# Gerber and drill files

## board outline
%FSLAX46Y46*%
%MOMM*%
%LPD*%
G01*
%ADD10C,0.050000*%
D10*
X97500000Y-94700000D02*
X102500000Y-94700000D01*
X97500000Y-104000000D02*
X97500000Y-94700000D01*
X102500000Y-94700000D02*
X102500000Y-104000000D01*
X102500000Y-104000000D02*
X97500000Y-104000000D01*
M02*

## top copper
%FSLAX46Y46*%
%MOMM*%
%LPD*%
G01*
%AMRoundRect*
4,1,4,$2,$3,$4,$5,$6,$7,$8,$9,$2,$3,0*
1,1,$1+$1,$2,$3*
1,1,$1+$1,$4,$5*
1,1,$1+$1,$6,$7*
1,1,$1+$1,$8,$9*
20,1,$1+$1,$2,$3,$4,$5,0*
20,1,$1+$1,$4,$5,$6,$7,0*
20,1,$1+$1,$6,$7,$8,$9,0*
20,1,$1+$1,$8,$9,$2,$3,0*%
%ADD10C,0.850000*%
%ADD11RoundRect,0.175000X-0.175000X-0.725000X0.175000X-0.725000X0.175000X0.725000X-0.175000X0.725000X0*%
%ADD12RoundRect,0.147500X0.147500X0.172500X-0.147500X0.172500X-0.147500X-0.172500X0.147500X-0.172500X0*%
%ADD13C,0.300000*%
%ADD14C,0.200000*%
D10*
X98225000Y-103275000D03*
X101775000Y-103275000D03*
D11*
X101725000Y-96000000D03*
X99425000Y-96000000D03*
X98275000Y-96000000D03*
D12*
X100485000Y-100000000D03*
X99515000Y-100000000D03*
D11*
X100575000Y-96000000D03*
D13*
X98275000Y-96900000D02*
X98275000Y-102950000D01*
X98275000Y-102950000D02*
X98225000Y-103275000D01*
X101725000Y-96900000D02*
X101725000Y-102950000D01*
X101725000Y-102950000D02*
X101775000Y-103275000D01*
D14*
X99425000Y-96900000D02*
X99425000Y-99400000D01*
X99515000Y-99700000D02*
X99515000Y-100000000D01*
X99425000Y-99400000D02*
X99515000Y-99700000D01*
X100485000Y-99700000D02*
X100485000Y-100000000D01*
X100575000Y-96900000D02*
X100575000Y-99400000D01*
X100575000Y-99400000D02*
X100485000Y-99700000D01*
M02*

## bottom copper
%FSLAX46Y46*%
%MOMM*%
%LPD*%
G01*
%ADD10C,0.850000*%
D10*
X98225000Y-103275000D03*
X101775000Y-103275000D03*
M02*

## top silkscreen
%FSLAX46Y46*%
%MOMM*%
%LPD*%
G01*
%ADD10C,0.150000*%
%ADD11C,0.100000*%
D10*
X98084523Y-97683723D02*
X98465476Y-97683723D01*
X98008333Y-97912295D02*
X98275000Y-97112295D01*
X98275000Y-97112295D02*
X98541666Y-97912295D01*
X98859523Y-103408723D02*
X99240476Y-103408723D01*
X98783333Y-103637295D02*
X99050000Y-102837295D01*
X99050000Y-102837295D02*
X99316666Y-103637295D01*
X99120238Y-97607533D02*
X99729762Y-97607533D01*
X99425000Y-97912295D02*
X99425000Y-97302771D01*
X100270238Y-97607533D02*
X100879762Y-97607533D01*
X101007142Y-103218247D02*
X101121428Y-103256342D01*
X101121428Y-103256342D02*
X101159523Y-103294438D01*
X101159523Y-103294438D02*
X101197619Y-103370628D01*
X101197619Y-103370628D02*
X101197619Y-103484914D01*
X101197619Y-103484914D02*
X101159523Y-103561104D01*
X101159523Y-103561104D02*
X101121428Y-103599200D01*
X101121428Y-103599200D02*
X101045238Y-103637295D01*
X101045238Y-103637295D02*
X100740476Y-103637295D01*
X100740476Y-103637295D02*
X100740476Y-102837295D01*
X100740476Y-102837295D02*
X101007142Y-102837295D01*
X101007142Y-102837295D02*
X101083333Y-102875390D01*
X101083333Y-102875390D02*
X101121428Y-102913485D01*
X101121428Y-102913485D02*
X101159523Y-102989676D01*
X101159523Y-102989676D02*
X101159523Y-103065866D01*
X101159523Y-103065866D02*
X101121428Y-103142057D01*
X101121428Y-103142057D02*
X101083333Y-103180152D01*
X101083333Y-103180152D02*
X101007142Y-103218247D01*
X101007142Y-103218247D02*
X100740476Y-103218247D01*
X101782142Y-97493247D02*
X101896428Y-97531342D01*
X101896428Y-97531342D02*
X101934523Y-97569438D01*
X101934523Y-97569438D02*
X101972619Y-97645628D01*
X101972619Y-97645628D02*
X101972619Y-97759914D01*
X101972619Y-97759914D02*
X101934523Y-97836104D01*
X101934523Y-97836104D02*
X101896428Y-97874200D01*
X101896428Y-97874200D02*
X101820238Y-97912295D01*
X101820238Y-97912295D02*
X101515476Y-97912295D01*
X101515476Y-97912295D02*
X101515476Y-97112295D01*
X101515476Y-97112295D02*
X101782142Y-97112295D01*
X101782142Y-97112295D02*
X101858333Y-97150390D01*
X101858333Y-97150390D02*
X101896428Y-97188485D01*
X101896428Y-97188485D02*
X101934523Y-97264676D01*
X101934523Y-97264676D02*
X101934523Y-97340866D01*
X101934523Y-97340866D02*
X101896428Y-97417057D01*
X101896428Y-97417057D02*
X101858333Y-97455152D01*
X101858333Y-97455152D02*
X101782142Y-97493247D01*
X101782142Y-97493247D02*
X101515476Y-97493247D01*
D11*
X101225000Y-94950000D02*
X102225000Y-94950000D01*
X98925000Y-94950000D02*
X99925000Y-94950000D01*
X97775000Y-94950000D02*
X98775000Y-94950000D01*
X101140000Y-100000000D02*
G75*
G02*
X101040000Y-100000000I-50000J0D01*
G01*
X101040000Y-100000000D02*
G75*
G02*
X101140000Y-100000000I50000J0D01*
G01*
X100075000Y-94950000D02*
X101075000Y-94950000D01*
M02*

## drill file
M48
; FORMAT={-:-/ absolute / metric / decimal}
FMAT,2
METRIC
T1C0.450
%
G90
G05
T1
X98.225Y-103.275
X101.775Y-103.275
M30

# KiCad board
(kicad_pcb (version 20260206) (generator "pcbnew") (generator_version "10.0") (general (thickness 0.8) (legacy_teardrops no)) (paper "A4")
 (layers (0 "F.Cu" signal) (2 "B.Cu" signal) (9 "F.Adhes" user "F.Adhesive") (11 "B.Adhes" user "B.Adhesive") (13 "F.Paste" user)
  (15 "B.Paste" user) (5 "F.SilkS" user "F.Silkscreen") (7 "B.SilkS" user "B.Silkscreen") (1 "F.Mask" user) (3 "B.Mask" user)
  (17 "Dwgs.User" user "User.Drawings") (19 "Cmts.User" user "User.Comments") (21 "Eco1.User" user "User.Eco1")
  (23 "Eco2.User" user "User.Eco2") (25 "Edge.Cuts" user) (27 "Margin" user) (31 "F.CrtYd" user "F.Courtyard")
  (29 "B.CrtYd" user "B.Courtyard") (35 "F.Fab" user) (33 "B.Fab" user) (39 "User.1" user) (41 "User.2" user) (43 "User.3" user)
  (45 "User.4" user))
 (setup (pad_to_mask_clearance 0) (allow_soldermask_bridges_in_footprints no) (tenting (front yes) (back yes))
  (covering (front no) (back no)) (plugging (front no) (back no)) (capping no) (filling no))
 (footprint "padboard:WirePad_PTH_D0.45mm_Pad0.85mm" (layer "F.Cu") (at 98.225 103.275)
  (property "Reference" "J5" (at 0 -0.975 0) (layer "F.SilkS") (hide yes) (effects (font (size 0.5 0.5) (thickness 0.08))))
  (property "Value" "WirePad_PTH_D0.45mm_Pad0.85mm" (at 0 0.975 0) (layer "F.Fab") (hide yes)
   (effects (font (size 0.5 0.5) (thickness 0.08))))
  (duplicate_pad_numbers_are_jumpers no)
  (pad "1" thru_hole circle (at 0 0) (size 0.85 0.85) (drill 0.45) (layers "*.Cu" "*.Mask") (remove_unused_layers no) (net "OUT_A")))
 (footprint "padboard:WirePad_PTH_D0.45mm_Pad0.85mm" (layer "F.Cu") (at 101.775 103.275)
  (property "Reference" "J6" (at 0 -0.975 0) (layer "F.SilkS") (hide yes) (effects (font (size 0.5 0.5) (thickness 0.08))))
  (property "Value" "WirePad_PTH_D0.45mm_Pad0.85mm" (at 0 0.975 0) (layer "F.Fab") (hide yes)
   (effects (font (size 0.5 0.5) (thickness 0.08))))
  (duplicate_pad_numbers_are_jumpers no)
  (pad "1" thru_hole circle (at 0 0) (size 0.85 0.85) (drill 0.45) (layers "*.Cu" "*.Mask") (remove_unused_layers no) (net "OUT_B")))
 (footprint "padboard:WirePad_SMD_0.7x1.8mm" (layer "F.Cu") (at 101.725 96)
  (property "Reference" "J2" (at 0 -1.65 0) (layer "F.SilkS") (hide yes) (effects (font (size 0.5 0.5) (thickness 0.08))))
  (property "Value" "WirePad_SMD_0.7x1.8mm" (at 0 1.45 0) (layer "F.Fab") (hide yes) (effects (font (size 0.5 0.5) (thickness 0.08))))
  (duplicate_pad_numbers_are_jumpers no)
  (fp_line (start -0.5 -1.05) (end 0.5 -1.05) (stroke (width 0.1) (type solid)) (layer "F.SilkS"))
  (pad "1" smd roundrect (at 0 0) (size 0.7 1.8) (layers "F.Cu" "F.Mask" "F.Paste") (roundrect_rratio 0.25) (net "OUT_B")))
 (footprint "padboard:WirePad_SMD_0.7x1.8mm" (layer "F.Cu") (at 99.425 96)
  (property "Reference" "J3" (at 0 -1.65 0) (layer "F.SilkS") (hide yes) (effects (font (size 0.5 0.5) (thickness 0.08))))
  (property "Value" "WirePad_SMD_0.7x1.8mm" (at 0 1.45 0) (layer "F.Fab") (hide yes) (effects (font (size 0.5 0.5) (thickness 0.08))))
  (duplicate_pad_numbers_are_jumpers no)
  (fp_line (start -0.5 -1.05) (end 0.5 -1.05) (stroke (width 0.1) (type solid)) (layer "F.SilkS"))
  (pad "1" smd roundrect (at 0 0) (size 0.7 1.8) (layers "F.Cu" "F.Mask" "F.Paste") (roundrect_rratio 0.25) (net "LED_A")))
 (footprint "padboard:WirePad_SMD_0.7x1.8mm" (layer "F.Cu") (at 98.275 96)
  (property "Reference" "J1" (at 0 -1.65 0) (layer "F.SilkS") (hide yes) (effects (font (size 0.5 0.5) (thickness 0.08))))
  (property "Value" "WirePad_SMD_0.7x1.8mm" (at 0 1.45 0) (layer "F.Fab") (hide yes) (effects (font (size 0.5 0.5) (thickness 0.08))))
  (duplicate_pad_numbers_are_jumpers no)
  (fp_line (start -0.5 -1.05) (end 0.5 -1.05) (stroke (width 0.1) (type solid)) (layer "F.SilkS"))
  (pad "1" smd roundrect (at 0 0) (size 0.7 1.8) (layers "F.Cu" "F.Mask" "F.Paste") (roundrect_rratio 0.25) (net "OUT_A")))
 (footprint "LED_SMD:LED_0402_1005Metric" (layer "F.Cu") (at 100 100 180)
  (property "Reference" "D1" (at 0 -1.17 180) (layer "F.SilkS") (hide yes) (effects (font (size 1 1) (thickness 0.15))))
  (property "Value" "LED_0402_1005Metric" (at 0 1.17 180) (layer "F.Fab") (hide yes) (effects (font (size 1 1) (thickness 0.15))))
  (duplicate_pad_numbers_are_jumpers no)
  (fp_circle (center -1.09 0) (end -1.04 0) (stroke (width 0.1) (type solid)) (fill no) (layer "F.SilkS"))
  (pad "1" smd roundrect (at -0.485 0 180) (size 0.59 0.64) (layers "F.Cu" "F.Mask" "F.Paste") (roundrect_rratio 0.25) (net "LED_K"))
  (pad "2" smd roundrect (at 0.485 0 180) (size 0.59 0.64) (layers "F.Cu" "F.Mask" "F.Paste") (roundrect_rratio 0.25) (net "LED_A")))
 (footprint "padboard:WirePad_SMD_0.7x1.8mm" (layer "F.Cu") (at 100.575 96)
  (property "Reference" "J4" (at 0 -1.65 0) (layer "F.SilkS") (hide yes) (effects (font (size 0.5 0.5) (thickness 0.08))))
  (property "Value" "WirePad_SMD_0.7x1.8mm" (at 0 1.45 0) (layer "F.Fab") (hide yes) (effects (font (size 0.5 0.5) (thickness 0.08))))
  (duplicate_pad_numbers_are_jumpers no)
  (fp_line (start -0.5 -1.05) (end 0.5 -1.05) (stroke (width 0.1) (type solid)) (layer "F.SilkS"))
  (pad "1" smd roundrect (at 0 0) (size 0.7 1.8) (layers "F.Cu" "F.Mask" "F.Paste") (roundrect_rratio 0.25) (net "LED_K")))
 (gr_line (start 97.5 94.7) (end 102.5 94.7) (stroke (width 0.05) (type default)) (layer "Edge.Cuts"))
 (gr_line (start 97.5 104) (end 97.5 94.7) (stroke (width 0.05) (type default)) (layer "Edge.Cuts"))
 (gr_line (start 102.5 94.7) (end 102.5 104) (stroke (width 0.05) (type default)) (layer "Edge.Cuts"))
 (gr_line (start 102.5 104) (end 97.5 104) (stroke (width 0.05) (type default)) (layer "Edge.Cuts"))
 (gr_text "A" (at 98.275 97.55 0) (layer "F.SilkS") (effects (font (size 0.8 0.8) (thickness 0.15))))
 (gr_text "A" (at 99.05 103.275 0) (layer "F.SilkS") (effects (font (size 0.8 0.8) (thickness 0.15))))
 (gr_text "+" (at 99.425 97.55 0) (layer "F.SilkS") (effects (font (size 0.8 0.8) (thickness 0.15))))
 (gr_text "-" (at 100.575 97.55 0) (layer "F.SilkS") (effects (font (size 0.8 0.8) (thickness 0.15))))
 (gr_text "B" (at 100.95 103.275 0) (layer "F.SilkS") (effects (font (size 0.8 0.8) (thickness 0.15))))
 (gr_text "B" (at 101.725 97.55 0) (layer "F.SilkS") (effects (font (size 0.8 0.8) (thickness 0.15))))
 (segment (start 98.275 96.9) (end 98.275 102.95) (width 0.3) (layer "F.Cu") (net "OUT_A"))
 (segment (start 98.275 102.95) (end 98.225 103.275) (width 0.3) (layer "F.Cu") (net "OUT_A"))
 (segment (start 101.725 96.9) (end 101.725 102.95) (width 0.3) (layer "F.Cu") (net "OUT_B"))
 (segment (start 101.725 102.95) (end 101.775 103.275) (width 0.3) (layer "F.Cu") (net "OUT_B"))
 (segment (start 99.425 96.9) (end 99.425 99.4) (width 0.2) (layer "F.Cu") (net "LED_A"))
 (segment (start 99.515 99.7) (end 99.515 100) (width 0.2) (layer "F.Cu") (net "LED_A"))
 (segment (start 99.425 99.4) (end 99.515 99.7) (width 0.2) (layer "F.Cu") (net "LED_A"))
 (segment (start 100.485 99.7) (end 100.485 100) (width 0.2) (layer "F.Cu") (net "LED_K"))
 (segment (start 100.575 96.9) (end 100.575 99.4) (width 0.2) (layer "F.Cu") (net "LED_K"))
 (segment (start 100.575 99.4) (end 100.485 99.7) (width 0.2) (layer "F.Cu") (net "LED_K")))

